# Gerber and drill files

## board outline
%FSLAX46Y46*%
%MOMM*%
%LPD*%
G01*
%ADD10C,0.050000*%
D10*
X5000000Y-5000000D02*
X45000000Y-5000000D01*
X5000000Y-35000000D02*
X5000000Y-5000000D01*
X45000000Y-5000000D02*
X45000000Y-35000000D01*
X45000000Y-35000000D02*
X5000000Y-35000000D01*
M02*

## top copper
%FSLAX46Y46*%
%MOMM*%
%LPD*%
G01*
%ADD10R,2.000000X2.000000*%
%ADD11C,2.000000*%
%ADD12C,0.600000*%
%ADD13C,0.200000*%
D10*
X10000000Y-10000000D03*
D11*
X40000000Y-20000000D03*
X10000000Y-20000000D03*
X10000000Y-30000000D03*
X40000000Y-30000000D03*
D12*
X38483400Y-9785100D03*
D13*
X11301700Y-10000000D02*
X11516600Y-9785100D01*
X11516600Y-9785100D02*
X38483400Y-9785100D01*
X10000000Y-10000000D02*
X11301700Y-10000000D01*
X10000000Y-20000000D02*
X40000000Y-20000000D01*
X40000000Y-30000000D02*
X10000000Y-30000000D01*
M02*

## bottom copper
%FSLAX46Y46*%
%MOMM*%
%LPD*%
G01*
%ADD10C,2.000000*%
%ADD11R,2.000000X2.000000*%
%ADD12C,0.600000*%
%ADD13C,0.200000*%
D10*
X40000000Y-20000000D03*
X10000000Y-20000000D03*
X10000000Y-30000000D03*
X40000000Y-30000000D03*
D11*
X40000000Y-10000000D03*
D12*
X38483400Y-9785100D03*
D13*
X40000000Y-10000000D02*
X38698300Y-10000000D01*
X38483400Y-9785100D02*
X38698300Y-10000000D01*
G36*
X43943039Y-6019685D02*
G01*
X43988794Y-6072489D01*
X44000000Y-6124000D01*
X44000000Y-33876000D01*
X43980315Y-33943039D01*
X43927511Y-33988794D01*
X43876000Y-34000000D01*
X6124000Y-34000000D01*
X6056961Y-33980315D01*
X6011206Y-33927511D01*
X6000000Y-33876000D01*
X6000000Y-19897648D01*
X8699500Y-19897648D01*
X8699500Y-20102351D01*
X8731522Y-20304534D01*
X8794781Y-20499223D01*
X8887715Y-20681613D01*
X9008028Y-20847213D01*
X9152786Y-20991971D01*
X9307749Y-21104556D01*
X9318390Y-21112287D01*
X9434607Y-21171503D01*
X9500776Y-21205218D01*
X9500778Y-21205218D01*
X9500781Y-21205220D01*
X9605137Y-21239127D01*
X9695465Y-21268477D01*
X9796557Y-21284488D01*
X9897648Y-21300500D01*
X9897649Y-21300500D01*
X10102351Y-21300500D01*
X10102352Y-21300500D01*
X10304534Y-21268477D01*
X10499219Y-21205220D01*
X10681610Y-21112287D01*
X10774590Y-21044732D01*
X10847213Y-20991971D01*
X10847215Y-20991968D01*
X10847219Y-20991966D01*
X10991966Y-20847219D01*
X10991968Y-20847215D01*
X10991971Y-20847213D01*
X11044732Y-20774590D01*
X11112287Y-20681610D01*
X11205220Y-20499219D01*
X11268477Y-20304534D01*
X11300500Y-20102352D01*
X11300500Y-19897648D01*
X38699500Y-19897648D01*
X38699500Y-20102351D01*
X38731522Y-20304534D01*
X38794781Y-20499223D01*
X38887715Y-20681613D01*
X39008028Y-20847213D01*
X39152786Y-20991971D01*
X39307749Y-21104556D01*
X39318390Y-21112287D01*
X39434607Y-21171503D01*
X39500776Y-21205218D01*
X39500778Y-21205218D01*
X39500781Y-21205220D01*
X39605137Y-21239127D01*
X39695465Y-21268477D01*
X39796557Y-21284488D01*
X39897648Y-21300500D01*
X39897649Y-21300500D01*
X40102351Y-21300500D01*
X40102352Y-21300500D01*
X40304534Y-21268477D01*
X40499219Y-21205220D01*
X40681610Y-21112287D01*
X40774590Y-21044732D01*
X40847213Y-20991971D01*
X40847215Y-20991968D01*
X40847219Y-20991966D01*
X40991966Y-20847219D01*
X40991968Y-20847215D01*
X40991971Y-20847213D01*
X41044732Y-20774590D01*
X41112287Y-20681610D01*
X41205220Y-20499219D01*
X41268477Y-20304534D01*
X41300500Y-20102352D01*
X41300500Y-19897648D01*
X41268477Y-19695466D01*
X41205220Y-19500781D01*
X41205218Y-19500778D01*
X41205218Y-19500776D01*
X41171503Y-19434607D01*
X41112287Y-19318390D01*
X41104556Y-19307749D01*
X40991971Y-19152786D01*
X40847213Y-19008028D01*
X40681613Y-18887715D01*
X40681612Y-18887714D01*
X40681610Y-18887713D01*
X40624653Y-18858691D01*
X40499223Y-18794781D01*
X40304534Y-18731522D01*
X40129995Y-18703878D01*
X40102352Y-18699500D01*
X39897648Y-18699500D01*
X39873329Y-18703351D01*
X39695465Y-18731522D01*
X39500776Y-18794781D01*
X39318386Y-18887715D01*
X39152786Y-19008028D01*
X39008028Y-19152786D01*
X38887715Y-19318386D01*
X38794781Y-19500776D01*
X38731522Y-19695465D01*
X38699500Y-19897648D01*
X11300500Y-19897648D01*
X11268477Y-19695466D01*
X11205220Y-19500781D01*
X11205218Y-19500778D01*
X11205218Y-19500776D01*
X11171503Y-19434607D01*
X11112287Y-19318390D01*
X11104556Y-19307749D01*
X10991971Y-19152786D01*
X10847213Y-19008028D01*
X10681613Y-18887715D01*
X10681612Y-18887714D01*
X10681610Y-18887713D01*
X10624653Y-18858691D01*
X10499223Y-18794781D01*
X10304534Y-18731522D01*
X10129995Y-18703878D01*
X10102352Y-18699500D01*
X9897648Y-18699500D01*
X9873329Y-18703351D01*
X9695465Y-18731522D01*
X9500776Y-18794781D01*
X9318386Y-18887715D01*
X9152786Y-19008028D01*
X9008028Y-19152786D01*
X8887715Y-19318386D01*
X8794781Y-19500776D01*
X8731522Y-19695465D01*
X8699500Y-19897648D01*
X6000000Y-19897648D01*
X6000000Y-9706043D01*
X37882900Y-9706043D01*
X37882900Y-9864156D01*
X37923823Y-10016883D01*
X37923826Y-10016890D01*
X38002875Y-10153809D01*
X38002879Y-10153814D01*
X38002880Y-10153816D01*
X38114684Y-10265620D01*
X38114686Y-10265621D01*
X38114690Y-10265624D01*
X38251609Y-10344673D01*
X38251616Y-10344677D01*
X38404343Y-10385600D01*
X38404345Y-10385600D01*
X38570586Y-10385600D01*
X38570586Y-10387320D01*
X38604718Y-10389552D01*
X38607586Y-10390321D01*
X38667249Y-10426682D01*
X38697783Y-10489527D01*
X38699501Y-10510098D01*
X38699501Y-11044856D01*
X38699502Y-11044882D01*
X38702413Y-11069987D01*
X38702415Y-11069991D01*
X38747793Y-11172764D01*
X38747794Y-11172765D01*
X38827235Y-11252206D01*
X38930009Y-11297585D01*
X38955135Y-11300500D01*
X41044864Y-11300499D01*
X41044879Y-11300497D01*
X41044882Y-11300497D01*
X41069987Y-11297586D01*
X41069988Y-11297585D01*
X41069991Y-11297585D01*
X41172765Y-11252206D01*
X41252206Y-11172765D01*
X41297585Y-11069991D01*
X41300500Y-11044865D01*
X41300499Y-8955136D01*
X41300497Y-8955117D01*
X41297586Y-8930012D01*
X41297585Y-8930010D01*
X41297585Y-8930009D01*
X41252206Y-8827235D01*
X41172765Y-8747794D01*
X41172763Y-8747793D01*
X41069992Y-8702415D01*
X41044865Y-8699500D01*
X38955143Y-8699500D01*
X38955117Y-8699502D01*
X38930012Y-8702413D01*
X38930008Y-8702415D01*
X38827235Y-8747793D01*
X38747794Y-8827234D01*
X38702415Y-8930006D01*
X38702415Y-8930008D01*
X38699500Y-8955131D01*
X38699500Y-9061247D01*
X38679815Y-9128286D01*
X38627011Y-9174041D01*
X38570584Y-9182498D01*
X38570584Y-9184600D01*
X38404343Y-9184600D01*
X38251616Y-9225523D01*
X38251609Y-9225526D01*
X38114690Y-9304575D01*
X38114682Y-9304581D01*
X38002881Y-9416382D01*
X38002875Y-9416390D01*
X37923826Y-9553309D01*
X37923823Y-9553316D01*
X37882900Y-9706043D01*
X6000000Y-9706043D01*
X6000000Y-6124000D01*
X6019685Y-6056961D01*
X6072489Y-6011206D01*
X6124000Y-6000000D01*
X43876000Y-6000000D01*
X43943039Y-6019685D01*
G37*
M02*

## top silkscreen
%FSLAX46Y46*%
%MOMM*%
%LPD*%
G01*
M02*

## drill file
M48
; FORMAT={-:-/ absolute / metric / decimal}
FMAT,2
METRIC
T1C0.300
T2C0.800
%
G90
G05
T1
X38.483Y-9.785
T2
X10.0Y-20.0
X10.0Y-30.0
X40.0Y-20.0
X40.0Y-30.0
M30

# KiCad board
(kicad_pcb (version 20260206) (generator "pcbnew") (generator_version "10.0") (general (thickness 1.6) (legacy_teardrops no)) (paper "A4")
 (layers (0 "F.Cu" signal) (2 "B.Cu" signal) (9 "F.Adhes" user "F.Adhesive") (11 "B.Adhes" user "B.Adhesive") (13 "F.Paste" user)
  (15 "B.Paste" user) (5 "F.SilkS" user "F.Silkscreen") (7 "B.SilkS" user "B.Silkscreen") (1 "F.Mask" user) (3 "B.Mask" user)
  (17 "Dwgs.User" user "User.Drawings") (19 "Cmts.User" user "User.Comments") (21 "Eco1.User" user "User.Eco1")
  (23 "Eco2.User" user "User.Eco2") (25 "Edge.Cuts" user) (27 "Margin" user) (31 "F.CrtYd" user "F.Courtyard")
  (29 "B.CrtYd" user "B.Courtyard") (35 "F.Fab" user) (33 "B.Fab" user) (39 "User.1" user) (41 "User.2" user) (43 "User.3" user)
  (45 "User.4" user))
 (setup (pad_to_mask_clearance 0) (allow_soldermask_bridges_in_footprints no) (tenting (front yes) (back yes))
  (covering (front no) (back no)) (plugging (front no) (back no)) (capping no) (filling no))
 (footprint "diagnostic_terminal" (layer "F.Cu") (at 10 10)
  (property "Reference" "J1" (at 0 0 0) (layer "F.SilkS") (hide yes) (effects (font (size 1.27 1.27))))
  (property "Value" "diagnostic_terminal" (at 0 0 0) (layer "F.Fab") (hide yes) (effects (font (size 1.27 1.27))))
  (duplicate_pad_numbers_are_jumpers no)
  (pad "1" smd rect (at 0 0) (size 2 2) (layers "F.Cu") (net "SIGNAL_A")))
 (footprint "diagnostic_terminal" (layer "F.Cu") (at 40 20)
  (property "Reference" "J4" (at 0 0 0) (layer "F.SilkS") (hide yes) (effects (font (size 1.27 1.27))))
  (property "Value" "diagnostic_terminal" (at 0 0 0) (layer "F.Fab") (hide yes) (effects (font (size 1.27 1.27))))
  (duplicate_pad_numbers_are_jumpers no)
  (pad "1" thru_hole circle (at 0 0) (size 2 2) (drill 0.8) (layers "*.Cu") (remove_unused_layers no) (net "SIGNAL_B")))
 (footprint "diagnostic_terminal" (layer "F.Cu") (at 10 20)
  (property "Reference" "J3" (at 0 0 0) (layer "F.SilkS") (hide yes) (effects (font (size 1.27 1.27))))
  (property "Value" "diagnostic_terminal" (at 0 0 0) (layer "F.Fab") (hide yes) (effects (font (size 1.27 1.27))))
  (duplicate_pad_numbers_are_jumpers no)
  (pad "1" thru_hole circle (at 0 0) (size 2 2) (drill 0.8) (layers "*.Cu") (remove_unused_layers no) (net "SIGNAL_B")))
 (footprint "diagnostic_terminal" (layer "F.Cu") (at 10 30)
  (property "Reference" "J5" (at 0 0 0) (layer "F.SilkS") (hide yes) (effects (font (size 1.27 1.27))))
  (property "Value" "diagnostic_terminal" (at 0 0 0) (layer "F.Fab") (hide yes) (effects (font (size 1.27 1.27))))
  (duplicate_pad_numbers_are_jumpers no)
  (pad "1" thru_hole circle (at 0 0) (size 2 2) (drill 0.8) (layers "*.Cu") (remove_unused_layers no) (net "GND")))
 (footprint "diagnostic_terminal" (layer "F.Cu") (at 40 30)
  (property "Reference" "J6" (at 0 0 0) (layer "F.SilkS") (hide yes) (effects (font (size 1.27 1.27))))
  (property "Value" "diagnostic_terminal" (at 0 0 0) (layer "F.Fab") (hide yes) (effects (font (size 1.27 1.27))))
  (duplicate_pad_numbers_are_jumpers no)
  (pad "1" thru_hole circle (at 0 0) (size 2 2) (drill 0.8) (layers "*.Cu") (remove_unused_layers no) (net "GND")))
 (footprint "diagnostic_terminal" (layer "B.Cu") (at 40 10)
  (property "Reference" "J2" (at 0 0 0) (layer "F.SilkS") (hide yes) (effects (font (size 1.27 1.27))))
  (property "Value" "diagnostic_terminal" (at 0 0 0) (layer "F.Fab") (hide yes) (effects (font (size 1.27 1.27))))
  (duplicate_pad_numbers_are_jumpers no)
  (pad "1" smd rect (at 0 0) (size 2 2) (layers "B.Cu") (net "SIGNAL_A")))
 (gr_line (start 5 5) (end 45 5) (stroke (width 0.05) (type default)) (layer "Edge.Cuts"))
 (gr_line (start 5 35) (end 5 5) (stroke (width 0.05) (type default)) (layer "Edge.Cuts"))
 (gr_line (start 45 5) (end 45 35) (stroke (width 0.05) (type default)) (layer "Edge.Cuts"))
 (gr_line (start 45 35) (end 5 35) (stroke (width 0.05) (type default)) (layer "Edge.Cuts"))
 (segment (start 11.3017 10) (end 11.5166 9.7851) (width 0.2) (layer "F.Cu") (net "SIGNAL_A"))
 (segment (start 11.5166 9.7851) (end 38.4834 9.7851) (width 0.2) (layer "F.Cu") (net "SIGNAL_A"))
 (segment (start 10 10) (end 11.3017 10) (width 0.2) (layer "F.Cu") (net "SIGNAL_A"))
 (via (at 38.4834 9.7851) (size 0.6) (drill 0.3) (layers "F.Cu" "B.Cu") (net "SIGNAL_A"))
 (segment (start 40 10) (end 38.6983 10) (width 0.2) (layer "B.Cu") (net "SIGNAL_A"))
 (segment (start 38.4834 9.7851) (end 38.6983 10) (width 0.2) (layer "B.Cu") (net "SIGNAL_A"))
 (segment (start 10 20) (end 40 20) (width 0.2) (layer "F.Cu") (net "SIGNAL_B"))
 (segment (start 40 30) (end 10 30) (width 0.2) (layer "F.Cu") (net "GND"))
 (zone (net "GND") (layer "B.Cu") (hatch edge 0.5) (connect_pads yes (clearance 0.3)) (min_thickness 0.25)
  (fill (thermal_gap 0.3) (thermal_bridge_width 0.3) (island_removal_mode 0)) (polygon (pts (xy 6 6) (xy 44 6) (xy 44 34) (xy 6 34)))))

